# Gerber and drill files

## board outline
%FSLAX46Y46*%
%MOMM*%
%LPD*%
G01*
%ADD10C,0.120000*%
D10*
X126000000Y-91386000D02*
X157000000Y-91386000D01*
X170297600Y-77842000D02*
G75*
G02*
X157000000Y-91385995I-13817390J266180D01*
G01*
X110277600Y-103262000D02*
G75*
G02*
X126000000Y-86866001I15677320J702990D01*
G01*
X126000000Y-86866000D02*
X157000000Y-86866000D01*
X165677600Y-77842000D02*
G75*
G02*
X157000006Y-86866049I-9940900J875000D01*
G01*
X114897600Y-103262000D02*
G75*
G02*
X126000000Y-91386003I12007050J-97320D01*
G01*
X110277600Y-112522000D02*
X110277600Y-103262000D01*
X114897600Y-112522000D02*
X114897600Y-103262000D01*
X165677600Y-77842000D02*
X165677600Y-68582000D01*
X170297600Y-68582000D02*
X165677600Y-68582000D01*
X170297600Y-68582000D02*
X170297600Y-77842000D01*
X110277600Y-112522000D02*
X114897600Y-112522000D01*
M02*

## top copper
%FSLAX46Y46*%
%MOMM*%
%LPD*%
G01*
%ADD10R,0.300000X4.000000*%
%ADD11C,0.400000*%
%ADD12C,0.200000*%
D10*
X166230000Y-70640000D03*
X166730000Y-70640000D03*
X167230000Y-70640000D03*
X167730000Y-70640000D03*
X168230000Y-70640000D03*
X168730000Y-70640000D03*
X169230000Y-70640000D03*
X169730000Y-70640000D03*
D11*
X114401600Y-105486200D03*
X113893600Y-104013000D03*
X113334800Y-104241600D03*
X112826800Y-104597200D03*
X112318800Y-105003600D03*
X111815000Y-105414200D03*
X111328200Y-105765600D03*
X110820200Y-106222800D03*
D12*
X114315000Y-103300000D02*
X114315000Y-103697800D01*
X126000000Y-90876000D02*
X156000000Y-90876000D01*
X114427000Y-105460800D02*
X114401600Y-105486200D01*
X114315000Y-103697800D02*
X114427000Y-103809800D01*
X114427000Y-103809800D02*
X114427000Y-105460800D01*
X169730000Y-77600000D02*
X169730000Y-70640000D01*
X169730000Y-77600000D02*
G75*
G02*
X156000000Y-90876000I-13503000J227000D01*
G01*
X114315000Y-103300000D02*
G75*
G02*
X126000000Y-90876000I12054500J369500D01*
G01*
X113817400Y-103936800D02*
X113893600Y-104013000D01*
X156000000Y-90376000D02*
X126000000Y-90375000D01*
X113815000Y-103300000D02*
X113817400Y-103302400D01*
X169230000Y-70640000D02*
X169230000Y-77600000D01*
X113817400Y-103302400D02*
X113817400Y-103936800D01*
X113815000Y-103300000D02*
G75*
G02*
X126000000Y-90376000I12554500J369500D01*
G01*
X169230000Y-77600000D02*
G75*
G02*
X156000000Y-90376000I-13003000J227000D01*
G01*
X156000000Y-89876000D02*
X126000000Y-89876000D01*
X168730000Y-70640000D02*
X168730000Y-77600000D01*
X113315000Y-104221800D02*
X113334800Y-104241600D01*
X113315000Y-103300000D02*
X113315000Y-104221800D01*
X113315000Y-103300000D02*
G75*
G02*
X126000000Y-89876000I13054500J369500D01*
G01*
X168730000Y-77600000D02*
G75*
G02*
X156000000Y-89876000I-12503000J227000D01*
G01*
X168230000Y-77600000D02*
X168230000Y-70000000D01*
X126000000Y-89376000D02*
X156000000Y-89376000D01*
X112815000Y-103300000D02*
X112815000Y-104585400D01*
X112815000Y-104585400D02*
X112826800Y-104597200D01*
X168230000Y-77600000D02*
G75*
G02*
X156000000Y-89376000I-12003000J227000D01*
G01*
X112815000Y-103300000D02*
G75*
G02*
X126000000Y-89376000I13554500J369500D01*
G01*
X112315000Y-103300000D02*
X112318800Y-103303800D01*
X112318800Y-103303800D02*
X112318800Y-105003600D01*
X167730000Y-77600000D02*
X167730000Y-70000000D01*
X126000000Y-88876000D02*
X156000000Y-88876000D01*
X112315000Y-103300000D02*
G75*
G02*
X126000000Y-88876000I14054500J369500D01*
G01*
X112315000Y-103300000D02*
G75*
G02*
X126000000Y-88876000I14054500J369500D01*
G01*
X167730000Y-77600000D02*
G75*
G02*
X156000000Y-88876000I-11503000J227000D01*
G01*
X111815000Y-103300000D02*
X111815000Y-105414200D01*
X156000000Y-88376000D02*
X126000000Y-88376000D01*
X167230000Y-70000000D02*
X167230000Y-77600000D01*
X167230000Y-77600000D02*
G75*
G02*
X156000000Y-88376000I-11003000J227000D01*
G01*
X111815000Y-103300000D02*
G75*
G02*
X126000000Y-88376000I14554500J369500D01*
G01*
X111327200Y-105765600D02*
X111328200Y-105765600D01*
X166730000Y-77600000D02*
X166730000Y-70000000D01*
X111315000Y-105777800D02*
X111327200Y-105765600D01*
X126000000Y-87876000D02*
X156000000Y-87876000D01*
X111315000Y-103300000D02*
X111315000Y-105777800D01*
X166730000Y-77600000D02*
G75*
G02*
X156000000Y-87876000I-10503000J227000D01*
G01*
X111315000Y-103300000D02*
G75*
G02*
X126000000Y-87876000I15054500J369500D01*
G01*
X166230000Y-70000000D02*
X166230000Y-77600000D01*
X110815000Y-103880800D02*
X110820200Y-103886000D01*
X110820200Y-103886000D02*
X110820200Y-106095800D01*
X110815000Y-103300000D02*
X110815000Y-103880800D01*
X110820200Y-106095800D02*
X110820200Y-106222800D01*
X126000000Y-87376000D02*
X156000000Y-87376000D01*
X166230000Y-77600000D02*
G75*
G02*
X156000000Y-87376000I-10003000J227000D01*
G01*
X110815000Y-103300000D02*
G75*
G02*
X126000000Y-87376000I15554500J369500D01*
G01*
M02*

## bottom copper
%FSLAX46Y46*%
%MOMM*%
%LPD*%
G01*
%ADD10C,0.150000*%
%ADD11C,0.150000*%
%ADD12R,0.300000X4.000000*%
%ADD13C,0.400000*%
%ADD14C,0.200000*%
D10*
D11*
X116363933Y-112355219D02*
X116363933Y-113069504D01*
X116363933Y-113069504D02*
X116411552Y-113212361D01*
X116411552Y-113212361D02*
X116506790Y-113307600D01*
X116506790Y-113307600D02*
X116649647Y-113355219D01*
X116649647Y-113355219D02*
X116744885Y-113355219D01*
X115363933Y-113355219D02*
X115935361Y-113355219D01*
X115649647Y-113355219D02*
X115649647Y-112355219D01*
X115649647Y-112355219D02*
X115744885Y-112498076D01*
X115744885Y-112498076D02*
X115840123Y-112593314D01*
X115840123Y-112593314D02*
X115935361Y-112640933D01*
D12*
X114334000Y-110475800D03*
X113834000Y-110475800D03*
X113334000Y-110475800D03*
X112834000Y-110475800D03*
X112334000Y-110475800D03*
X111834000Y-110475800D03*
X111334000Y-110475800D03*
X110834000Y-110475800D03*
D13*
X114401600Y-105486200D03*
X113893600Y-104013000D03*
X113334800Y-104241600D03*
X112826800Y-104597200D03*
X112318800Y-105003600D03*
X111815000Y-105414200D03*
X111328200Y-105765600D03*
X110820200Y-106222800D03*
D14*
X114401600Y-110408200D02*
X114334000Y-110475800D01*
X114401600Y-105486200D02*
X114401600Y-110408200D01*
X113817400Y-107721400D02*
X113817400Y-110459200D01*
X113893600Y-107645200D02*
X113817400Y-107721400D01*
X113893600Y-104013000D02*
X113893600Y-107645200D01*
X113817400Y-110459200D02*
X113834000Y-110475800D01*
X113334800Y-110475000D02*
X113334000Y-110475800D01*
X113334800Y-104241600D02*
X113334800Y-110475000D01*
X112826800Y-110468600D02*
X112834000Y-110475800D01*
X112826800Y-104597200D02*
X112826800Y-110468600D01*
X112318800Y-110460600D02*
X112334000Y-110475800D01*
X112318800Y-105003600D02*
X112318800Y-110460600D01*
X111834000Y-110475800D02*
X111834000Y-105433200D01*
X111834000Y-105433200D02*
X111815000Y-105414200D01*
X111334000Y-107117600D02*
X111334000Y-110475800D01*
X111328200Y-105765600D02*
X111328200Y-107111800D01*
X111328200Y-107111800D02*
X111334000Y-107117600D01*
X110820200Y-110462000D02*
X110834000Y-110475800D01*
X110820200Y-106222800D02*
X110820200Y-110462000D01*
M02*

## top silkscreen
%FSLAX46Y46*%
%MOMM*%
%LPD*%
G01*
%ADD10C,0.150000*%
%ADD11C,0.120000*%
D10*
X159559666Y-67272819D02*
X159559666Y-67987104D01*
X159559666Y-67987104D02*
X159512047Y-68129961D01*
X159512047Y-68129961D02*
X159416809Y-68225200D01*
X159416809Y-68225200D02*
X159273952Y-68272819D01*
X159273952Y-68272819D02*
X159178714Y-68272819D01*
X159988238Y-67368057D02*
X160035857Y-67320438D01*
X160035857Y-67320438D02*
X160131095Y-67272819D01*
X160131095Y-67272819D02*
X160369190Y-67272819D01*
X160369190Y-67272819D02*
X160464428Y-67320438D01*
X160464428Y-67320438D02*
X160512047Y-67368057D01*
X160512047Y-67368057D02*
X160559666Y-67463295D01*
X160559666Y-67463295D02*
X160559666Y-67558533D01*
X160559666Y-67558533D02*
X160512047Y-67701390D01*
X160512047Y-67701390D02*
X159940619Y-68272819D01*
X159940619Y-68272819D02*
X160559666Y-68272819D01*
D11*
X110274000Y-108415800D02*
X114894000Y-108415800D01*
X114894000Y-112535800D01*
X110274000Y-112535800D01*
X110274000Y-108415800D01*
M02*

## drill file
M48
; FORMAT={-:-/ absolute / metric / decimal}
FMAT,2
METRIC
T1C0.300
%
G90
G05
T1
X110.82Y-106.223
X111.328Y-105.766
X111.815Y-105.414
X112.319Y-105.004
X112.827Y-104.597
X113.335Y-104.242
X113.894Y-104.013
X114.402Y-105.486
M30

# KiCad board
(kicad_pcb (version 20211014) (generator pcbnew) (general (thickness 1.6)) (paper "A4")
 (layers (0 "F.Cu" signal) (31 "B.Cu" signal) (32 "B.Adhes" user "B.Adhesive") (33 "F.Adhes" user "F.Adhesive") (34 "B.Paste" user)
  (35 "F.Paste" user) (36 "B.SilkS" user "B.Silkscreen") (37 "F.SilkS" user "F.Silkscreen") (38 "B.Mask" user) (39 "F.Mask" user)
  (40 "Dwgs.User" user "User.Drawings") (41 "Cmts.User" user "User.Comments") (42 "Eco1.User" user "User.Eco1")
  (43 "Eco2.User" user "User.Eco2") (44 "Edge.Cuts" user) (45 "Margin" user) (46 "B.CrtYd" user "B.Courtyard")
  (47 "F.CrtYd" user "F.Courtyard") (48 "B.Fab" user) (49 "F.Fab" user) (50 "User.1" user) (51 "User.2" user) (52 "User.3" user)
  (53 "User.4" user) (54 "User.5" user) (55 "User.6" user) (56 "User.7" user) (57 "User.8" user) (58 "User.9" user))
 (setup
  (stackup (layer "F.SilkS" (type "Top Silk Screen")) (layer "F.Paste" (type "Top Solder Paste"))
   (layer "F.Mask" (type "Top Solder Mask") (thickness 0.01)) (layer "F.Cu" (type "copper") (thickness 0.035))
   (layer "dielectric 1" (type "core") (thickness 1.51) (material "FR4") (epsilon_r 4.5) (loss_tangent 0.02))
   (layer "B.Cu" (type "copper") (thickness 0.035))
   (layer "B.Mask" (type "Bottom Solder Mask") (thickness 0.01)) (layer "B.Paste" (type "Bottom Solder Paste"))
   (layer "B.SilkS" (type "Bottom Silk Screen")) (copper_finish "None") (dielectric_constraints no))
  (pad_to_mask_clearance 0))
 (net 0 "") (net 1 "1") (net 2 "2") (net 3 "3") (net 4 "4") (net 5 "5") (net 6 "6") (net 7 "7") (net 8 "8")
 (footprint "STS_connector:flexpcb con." (layer "F.Cu") (at 165.73 72.64)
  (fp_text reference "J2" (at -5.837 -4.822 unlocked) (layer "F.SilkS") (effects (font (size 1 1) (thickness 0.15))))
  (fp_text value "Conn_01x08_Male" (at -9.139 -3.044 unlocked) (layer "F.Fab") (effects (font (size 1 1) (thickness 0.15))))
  (pad "1" smd rect (at 0.5 -2) (size 0.3 4) (layers "F.Cu" "F.Paste" "F.Mask") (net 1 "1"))
  (pad "2" smd rect (at 1 -2) (size 0.3 4) (layers "F.Cu" "F.Paste" "F.Mask") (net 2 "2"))
  (pad "3" smd rect (at 1.5 -2) (size 0.3 4) (layers "F.Cu" "F.Paste" "F.Mask") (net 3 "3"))
  (pad "4" smd rect (at 2 -2) (size 0.3 4) (layers "F.Cu" "F.Paste" "F.Mask") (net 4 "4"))
  (pad "5" smd rect (at 2.5 -2) (size 0.3 4) (layers "F.Cu" "F.Paste" "F.Mask") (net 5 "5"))
  (pad "6" smd rect (at 3 -2) (size 0.3 4) (layers "F.Cu" "F.Paste" "F.Mask") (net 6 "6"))
  (pad "7" smd rect (at 3.5 -2) (size 0.3 4) (layers "F.Cu" "F.Paste" "F.Mask") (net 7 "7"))
  (pad "8" smd rect (at 4 -2) (size 0.3 4) (layers "F.Cu" "F.Paste" "F.Mask") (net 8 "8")))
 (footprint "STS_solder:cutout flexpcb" (layer "F.Cu") (at 110.3376 112.522)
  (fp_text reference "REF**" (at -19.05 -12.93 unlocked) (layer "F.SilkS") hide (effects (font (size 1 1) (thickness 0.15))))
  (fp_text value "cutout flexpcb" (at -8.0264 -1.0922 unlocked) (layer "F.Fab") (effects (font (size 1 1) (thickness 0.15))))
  (fp_line (start -0.06 0) (end -0.06 -9.26) (layer "Edge.Cuts") (width 0.12))
  (fp_line (start 4.56 0) (end 4.56 -9.26) (layer "Edge.Cuts") (width 0.12))
  (fp_line (start 55.34 -34.68) (end 55.34 -43.94) (layer "Edge.Cuts") (width 0.12))
  (fp_line (start 59.96 -43.94) (end 55.34 -43.94) (layer "Edge.Cuts") (width 0.12))
  (fp_line (start 59.96 -43.94) (end 59.96 -34.68) (layer "Edge.Cuts") (width 0.12))
  (fp_line (start -0.06 0) (end 4.56 0) (layer "Edge.Cuts") (width 0.12)))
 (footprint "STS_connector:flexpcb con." (layer "B.Cu") (at 114.834 112.4758 180)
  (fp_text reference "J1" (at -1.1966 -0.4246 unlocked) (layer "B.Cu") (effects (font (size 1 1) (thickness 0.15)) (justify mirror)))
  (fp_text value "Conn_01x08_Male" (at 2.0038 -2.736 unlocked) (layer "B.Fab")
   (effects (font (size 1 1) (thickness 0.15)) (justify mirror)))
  (fp_rect (start -0.06 -0.06) (end 4.56 4.06) (layer "F.SilkS") (width 0.12) (fill none))
  (pad "1" smd rect (at 0.5 2 180) (size 0.3 4) (layers "B.Cu" "B.Paste" "B.Mask") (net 8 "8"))
  (pad "2" smd rect (at 1 2 180) (size 0.3 4) (layers "B.Cu" "B.Paste" "B.Mask") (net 7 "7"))
  (pad "3" smd rect (at 1.5 2 180) (size 0.3 4) (layers "B.Cu" "B.Paste" "B.Mask") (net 6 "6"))
  (pad "4" smd rect (at 2 2 180) (size 0.3 4) (layers "B.Cu" "B.Paste" "B.Mask") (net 5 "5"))
  (pad "5" smd rect (at 2.5 2 180) (size 0.3 4) (layers "B.Cu" "B.Paste" "B.Mask") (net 4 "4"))
  (pad "6" smd rect (at 3 2 180) (size 0.3 4) (layers "B.Cu" "B.Paste" "B.Mask") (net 3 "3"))
  (pad "7" smd rect (at 3.5 2 180) (size 0.3 4) (layers "B.Cu" "B.Paste" "B.Mask") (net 2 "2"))
  (pad "8" smd rect (at 4 2 180) (size 0.3 4) (layers "B.Cu" "B.Paste" "B.Mask") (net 1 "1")))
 (gr_line (start 126 91.386) (end 157 91.386) (layer "Edge.Cuts") (width 0.12))
 (gr_arc (start 170.2976 77.842) (mid 166.341683 87.257893) (end 157 91.386) (layer "Edge.Cuts") (width 0.12))
 (gr_arc (start 110.2776 103.262) (mid 114.628009 91.697444) (end 126 86.866) (layer "Edge.Cuts") (width 0.12))
 (gr_line (start 126 86.866) (end 157 86.866) (layer "Edge.Cuts") (width 0.12))
 (gr_arc (start 165.6776 77.842) (mid 162.929877 83.884001) (end 157 86.866) (layer "Edge.Cuts") (width 0.12))
 (gr_arc (start 114.8976 103.262) (mid 118.133228 95.159264) (end 126 91.386) (layer "Edge.Cuts") (width 0.12))
 (segment (start 114.315 103.3) (end 114.315 103.6978) (width 0.2) (layer "F.Cu") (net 8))
 (segment (start 126 90.876) (end 156 90.876) (width 0.2) (layer "F.Cu") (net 8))
 (segment (start 114.427 105.4608) (end 114.4016 105.4862) (width 0.2) (layer "F.Cu") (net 8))
 (segment (start 114.315 103.6978) (end 114.427 103.8098) (width 0.2) (layer "F.Cu") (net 8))
 (segment (start 114.427 103.8098) (end 114.427 105.4608) (width 0.2) (layer "F.Cu") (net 8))
 (segment (start 169.73 77.6) (end 169.73 70.64) (width 0.2) (layer "F.Cu") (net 8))
 (via (at 114.4016 105.4862) (size 0.4) (drill 0.3) (layers "F.Cu" "B.Cu") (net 8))
 (arc (start 169.73 77.6) (mid 165.61455 87.081577) (end 156 90.876) (width 0.2) (layer "F.Cu") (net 8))
 (arc (start 114.315 103.3) (mid 117.584405 94.667957) (end 126 90.876) (width 0.2) (layer "F.Cu") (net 8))
 (segment (start 114.4016 110.4082) (end 114.334 110.4758) (width 0.2) (layer "B.Cu") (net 8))
 (segment (start 114.4016 105.4862) (end 114.4016 110.4082) (width 0.2) (layer "B.Cu") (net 8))
 (segment (start 113.8174 103.9368) (end 113.8936 104.013) (width 0.2) (layer "F.Cu") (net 7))
 (segment (start 156 90.376) (end 126 90.375) (width 0.2) (layer "F.Cu") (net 7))
 (segment (start 113.815 103.3) (end 113.8174 103.3024) (width 0.2) (layer "F.Cu") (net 7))
 (segment (start 169.23 70.64) (end 169.23 77.6) (width 0.2) (layer "F.Cu") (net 7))
 (segment (start 113.8174 103.3024) (end 113.8174 103.9368) (width 0.2) (layer "F.Cu") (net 7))
 (via (at 113.8936 104.013) (size 0.4) (drill 0.3) (layers "F.Cu" "B.Cu") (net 7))
 (arc (start 113.815 103.3) (mid 117.230852 94.314404) (end 126 90.376) (width 0.2) (layer "F.Cu") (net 7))
 (arc (start 169.23 77.6) (mid 165.260997 86.728023) (end 156 90.376) (width 0.2) (layer "F.Cu") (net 7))
 (segment (start 113.8174 107.7214) (end 113.8174 110.4592) (width 0.2) (layer "B.Cu") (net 7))
 (segment (start 113.8936 107.6452) (end 113.8174 107.7214) (width 0.2) (layer "B.Cu") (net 7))
 (segment (start 113.8936 104.013) (end 113.8936 107.6452) (width 0.2) (layer "B.Cu") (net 7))
 (segment (start 113.8174 110.4592) (end 113.834 110.4758) (width 0.2) (layer "B.Cu") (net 7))
 (segment (start 156 89.876) (end 126 89.876) (width 0.2) (layer "F.Cu") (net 6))
 (segment (start 168.73 70.64) (end 168.73 77.6) (width 0.2) (layer "F.Cu") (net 6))
 (segment (start 113.315 104.2218) (end 113.3348 104.2416) (width 0.2) (layer "F.Cu") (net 6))
 (segment (start 113.315 103.3) (end 113.315 104.2218) (width 0.2) (layer "F.Cu") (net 6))
 (via (at 113.3348 104.2416) (size 0.4) (drill 0.3) (layers "F.Cu" "B.Cu") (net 6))
 (arc (start 113.315 103.3) (mid 116.877299 93.96085) (end 126 89.876) (width 0.2) (layer "F.Cu") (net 6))
 (arc (start 168.73 77.6) (mid 164.907443 86.374469) (end 156 89.876) (width 0.2) (layer "F.Cu") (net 6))
 (segment (start 113.3348 110.475) (end 113.334 110.4758) (width 0.2) (layer "B.Cu") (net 6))
 (segment (start 113.3348 104.2416) (end 113.3348 110.475) (width 0.2) (layer "B.Cu") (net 6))
 (segment (start 168.23 77.6) (end 168.23 70) (width 0.2) (layer "F.Cu") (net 5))
 (segment (start 126 89.376) (end 156 89.376) (width 0.2) (layer "F.Cu") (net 5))
 (segment (start 112.815 103.3) (end 112.815 104.5854) (width 0.2) (layer "F.Cu") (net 5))
 (segment (start 112.815 104.5854) (end 112.8268 104.5972) (width 0.2) (layer "F.Cu") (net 5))
 (via (at 112.8268 104.5972) (size 0.4) (drill 0.3) (layers "F.Cu" "B.Cu") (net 5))
 (arc (start 168.23 77.6) (mid 164.55389 86.020917) (end 156 89.376) (width 0.2) (layer "F.Cu") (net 5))
 (arc (start 112.815 103.3) (mid 116.523745 93.607297) (end 126 89.376) (width 0.2) (layer "F.Cu") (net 5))
 (segment (start 112.8268 110.4686) (end 112.834 110.4758) (width 0.2) (layer "B.Cu") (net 5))
 (segment (start 112.8268 104.5972) (end 112.8268 110.4686) (width 0.2) (layer "B.Cu") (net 5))
 (segment (start 112.315 103.3) (end 112.3188 103.3038) (width 0.2) (layer "F.Cu") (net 4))
 (segment (start 112.3188 103.3038) (end 112.3188 105.0036) (width 0.2) (layer "F.Cu") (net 4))
 (segment (start 167.73 77.6) (end 167.73 70) (width 0.2) (layer "F.Cu") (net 4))
 (segment (start 126 88.876) (end 156 88.876) (width 0.2) (layer "F.Cu") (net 4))
 (via (at 112.3188 105.0036) (size 0.4) (drill 0.3) (layers "F.Cu" "B.Cu") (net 4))
 (arc (start 112.315 103.3) (mid 116.170192 93.253744) (end 126 88.876) (width 0.2) (layer "F.Cu") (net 4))
 (arc (start 112.315 103.3) (mid 116.170192 93.253744) (end 126 88.876) (width 0.2) (layer "F.Cu") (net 4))
 (arc (start 167.73 77.6) (mid 164.200336 85.667363) (end 156 88.876) (width 0.2) (layer "F.Cu") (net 4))
 (segment (start 112.3188 110.4606) (end 112.334 110.4758) (width 0.2) (layer "B.Cu") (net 4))
 (segment (start 112.3188 105.0036) (end 112.3188 110.4606) (width 0.2) (layer "B.Cu") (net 4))
 (segment (start 111.815 103.3) (end 111.815 105.4142) (width 0.2) (layer "F.Cu") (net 3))
 (segment (start 156 88.376) (end 126 88.376) (width 0.2) (layer "F.Cu") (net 3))
 (segment (start 167.23 70) (end 167.23 77.6) (width 0.2) (layer "F.Cu") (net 3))
 (via (at 111.815 105.4142) (size 0.4) (drill 0.3) (layers "F.Cu" "B.Cu") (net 3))
 (arc (start 167.23 77.6) (mid 163.846783 85.313809) (end 156 88.376) (width 0.2) (layer "F.Cu") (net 3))
 (arc (start 111.815 103.3) (mid 115.816638 92.90019) (end 126 88.376) (width 0.2) (layer "F.Cu") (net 3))
 (segment (start 111.834 110.4758) (end 111.834 105.4332) (width 0.2) (layer "B.Cu") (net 3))
 (segment (start 111.834 105.4332) (end 111.815 105.4142) (width 0.2) (layer "B.Cu") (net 3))
 (segment (start 111.3272 105.7656) (end 111.3282 105.7656) (width 0.2) (layer "F.Cu") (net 2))
 (segment (start 166.73 77.6) (end 166.73 70) (width 0.2) (layer "F.Cu") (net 2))
 (segment (start 111.315 105.7778) (end 111.3272 105.7656) (width 0.2) (layer "F.Cu") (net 2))
 (segment (start 126 87.876) (end 156 87.876) (width 0.2) (layer "F.Cu") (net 2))
 (segment (start 111.315 103.3) (end 111.315 105.7778) (width 0.2) (layer "F.Cu") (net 2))
 (via (at 111.3282 105.7656) (size 0.4) (drill 0.3) (layers "F.Cu" "B.Cu") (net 2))
 (arc (start 166.73 77.6) (mid 163.493229 84.960256) (end 156 87.876) (width 0.2) (layer "F.Cu") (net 2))
 (arc (start 111.315 103.3) (mid 115.463085 92.546637) (end 126 87.876) (width 0.2) (layer "F.Cu") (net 2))
 (segment (start 111.334 107.1176) (end 111.334 110.4758) (width 0.2) (layer "B.Cu") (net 2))
 (segment (start 111.3282 105.7656) (end 111.3282 107.1118) (width 0.2) (layer "B.Cu") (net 2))
 (segment (start 111.3282 107.1118) (end 111.334 107.1176) (width 0.2) (layer "B.Cu") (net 2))
 (segment (start 166.23 70) (end 166.23 77.6) (width 0.2) (layer "F.Cu") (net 1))
 (segment (start 110.815 103.8808) (end 110.8202 103.886) (width 0.2) (layer "F.Cu") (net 1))
 (segment (start 110.8202 103.886) (end 110.8202 106.0958) (width 0.2) (layer "F.Cu") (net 1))
 (segment (start 110.815 103.3) (end 110.815 103.8808) (width 0.2) (layer "F.Cu") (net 1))
 (segment (start 110.8202 106.0958) (end 110.8202 106.2228) (width 0.2) (layer "F.Cu") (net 1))
 (segment (start 126 87.376) (end 156 87.376) (width 0.2) (layer "F.Cu") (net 1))
 (via (at 110.8202 106.2228) (size 0.4) (drill 0.3) (layers "F.Cu" "B.Cu") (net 1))
 (arc (start 166.23 77.6) (mid 163.139676 84.606702) (end 156 87.376) (width 0.2) (layer "F.Cu") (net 1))
 (arc (start 110.815 103.3) (mid 115.109532 92.193084) (end 126 87.376) (width 0.2) (layer "F.Cu") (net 1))
 (segment (start 110.8202 110.462) (end 110.834 110.4758) (width 0.2) (layer "B.Cu") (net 1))
 (segment (start 110.8202 106.2228) (end 110.8202 110.462) (width 0.2) (layer "B.Cu") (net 1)))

